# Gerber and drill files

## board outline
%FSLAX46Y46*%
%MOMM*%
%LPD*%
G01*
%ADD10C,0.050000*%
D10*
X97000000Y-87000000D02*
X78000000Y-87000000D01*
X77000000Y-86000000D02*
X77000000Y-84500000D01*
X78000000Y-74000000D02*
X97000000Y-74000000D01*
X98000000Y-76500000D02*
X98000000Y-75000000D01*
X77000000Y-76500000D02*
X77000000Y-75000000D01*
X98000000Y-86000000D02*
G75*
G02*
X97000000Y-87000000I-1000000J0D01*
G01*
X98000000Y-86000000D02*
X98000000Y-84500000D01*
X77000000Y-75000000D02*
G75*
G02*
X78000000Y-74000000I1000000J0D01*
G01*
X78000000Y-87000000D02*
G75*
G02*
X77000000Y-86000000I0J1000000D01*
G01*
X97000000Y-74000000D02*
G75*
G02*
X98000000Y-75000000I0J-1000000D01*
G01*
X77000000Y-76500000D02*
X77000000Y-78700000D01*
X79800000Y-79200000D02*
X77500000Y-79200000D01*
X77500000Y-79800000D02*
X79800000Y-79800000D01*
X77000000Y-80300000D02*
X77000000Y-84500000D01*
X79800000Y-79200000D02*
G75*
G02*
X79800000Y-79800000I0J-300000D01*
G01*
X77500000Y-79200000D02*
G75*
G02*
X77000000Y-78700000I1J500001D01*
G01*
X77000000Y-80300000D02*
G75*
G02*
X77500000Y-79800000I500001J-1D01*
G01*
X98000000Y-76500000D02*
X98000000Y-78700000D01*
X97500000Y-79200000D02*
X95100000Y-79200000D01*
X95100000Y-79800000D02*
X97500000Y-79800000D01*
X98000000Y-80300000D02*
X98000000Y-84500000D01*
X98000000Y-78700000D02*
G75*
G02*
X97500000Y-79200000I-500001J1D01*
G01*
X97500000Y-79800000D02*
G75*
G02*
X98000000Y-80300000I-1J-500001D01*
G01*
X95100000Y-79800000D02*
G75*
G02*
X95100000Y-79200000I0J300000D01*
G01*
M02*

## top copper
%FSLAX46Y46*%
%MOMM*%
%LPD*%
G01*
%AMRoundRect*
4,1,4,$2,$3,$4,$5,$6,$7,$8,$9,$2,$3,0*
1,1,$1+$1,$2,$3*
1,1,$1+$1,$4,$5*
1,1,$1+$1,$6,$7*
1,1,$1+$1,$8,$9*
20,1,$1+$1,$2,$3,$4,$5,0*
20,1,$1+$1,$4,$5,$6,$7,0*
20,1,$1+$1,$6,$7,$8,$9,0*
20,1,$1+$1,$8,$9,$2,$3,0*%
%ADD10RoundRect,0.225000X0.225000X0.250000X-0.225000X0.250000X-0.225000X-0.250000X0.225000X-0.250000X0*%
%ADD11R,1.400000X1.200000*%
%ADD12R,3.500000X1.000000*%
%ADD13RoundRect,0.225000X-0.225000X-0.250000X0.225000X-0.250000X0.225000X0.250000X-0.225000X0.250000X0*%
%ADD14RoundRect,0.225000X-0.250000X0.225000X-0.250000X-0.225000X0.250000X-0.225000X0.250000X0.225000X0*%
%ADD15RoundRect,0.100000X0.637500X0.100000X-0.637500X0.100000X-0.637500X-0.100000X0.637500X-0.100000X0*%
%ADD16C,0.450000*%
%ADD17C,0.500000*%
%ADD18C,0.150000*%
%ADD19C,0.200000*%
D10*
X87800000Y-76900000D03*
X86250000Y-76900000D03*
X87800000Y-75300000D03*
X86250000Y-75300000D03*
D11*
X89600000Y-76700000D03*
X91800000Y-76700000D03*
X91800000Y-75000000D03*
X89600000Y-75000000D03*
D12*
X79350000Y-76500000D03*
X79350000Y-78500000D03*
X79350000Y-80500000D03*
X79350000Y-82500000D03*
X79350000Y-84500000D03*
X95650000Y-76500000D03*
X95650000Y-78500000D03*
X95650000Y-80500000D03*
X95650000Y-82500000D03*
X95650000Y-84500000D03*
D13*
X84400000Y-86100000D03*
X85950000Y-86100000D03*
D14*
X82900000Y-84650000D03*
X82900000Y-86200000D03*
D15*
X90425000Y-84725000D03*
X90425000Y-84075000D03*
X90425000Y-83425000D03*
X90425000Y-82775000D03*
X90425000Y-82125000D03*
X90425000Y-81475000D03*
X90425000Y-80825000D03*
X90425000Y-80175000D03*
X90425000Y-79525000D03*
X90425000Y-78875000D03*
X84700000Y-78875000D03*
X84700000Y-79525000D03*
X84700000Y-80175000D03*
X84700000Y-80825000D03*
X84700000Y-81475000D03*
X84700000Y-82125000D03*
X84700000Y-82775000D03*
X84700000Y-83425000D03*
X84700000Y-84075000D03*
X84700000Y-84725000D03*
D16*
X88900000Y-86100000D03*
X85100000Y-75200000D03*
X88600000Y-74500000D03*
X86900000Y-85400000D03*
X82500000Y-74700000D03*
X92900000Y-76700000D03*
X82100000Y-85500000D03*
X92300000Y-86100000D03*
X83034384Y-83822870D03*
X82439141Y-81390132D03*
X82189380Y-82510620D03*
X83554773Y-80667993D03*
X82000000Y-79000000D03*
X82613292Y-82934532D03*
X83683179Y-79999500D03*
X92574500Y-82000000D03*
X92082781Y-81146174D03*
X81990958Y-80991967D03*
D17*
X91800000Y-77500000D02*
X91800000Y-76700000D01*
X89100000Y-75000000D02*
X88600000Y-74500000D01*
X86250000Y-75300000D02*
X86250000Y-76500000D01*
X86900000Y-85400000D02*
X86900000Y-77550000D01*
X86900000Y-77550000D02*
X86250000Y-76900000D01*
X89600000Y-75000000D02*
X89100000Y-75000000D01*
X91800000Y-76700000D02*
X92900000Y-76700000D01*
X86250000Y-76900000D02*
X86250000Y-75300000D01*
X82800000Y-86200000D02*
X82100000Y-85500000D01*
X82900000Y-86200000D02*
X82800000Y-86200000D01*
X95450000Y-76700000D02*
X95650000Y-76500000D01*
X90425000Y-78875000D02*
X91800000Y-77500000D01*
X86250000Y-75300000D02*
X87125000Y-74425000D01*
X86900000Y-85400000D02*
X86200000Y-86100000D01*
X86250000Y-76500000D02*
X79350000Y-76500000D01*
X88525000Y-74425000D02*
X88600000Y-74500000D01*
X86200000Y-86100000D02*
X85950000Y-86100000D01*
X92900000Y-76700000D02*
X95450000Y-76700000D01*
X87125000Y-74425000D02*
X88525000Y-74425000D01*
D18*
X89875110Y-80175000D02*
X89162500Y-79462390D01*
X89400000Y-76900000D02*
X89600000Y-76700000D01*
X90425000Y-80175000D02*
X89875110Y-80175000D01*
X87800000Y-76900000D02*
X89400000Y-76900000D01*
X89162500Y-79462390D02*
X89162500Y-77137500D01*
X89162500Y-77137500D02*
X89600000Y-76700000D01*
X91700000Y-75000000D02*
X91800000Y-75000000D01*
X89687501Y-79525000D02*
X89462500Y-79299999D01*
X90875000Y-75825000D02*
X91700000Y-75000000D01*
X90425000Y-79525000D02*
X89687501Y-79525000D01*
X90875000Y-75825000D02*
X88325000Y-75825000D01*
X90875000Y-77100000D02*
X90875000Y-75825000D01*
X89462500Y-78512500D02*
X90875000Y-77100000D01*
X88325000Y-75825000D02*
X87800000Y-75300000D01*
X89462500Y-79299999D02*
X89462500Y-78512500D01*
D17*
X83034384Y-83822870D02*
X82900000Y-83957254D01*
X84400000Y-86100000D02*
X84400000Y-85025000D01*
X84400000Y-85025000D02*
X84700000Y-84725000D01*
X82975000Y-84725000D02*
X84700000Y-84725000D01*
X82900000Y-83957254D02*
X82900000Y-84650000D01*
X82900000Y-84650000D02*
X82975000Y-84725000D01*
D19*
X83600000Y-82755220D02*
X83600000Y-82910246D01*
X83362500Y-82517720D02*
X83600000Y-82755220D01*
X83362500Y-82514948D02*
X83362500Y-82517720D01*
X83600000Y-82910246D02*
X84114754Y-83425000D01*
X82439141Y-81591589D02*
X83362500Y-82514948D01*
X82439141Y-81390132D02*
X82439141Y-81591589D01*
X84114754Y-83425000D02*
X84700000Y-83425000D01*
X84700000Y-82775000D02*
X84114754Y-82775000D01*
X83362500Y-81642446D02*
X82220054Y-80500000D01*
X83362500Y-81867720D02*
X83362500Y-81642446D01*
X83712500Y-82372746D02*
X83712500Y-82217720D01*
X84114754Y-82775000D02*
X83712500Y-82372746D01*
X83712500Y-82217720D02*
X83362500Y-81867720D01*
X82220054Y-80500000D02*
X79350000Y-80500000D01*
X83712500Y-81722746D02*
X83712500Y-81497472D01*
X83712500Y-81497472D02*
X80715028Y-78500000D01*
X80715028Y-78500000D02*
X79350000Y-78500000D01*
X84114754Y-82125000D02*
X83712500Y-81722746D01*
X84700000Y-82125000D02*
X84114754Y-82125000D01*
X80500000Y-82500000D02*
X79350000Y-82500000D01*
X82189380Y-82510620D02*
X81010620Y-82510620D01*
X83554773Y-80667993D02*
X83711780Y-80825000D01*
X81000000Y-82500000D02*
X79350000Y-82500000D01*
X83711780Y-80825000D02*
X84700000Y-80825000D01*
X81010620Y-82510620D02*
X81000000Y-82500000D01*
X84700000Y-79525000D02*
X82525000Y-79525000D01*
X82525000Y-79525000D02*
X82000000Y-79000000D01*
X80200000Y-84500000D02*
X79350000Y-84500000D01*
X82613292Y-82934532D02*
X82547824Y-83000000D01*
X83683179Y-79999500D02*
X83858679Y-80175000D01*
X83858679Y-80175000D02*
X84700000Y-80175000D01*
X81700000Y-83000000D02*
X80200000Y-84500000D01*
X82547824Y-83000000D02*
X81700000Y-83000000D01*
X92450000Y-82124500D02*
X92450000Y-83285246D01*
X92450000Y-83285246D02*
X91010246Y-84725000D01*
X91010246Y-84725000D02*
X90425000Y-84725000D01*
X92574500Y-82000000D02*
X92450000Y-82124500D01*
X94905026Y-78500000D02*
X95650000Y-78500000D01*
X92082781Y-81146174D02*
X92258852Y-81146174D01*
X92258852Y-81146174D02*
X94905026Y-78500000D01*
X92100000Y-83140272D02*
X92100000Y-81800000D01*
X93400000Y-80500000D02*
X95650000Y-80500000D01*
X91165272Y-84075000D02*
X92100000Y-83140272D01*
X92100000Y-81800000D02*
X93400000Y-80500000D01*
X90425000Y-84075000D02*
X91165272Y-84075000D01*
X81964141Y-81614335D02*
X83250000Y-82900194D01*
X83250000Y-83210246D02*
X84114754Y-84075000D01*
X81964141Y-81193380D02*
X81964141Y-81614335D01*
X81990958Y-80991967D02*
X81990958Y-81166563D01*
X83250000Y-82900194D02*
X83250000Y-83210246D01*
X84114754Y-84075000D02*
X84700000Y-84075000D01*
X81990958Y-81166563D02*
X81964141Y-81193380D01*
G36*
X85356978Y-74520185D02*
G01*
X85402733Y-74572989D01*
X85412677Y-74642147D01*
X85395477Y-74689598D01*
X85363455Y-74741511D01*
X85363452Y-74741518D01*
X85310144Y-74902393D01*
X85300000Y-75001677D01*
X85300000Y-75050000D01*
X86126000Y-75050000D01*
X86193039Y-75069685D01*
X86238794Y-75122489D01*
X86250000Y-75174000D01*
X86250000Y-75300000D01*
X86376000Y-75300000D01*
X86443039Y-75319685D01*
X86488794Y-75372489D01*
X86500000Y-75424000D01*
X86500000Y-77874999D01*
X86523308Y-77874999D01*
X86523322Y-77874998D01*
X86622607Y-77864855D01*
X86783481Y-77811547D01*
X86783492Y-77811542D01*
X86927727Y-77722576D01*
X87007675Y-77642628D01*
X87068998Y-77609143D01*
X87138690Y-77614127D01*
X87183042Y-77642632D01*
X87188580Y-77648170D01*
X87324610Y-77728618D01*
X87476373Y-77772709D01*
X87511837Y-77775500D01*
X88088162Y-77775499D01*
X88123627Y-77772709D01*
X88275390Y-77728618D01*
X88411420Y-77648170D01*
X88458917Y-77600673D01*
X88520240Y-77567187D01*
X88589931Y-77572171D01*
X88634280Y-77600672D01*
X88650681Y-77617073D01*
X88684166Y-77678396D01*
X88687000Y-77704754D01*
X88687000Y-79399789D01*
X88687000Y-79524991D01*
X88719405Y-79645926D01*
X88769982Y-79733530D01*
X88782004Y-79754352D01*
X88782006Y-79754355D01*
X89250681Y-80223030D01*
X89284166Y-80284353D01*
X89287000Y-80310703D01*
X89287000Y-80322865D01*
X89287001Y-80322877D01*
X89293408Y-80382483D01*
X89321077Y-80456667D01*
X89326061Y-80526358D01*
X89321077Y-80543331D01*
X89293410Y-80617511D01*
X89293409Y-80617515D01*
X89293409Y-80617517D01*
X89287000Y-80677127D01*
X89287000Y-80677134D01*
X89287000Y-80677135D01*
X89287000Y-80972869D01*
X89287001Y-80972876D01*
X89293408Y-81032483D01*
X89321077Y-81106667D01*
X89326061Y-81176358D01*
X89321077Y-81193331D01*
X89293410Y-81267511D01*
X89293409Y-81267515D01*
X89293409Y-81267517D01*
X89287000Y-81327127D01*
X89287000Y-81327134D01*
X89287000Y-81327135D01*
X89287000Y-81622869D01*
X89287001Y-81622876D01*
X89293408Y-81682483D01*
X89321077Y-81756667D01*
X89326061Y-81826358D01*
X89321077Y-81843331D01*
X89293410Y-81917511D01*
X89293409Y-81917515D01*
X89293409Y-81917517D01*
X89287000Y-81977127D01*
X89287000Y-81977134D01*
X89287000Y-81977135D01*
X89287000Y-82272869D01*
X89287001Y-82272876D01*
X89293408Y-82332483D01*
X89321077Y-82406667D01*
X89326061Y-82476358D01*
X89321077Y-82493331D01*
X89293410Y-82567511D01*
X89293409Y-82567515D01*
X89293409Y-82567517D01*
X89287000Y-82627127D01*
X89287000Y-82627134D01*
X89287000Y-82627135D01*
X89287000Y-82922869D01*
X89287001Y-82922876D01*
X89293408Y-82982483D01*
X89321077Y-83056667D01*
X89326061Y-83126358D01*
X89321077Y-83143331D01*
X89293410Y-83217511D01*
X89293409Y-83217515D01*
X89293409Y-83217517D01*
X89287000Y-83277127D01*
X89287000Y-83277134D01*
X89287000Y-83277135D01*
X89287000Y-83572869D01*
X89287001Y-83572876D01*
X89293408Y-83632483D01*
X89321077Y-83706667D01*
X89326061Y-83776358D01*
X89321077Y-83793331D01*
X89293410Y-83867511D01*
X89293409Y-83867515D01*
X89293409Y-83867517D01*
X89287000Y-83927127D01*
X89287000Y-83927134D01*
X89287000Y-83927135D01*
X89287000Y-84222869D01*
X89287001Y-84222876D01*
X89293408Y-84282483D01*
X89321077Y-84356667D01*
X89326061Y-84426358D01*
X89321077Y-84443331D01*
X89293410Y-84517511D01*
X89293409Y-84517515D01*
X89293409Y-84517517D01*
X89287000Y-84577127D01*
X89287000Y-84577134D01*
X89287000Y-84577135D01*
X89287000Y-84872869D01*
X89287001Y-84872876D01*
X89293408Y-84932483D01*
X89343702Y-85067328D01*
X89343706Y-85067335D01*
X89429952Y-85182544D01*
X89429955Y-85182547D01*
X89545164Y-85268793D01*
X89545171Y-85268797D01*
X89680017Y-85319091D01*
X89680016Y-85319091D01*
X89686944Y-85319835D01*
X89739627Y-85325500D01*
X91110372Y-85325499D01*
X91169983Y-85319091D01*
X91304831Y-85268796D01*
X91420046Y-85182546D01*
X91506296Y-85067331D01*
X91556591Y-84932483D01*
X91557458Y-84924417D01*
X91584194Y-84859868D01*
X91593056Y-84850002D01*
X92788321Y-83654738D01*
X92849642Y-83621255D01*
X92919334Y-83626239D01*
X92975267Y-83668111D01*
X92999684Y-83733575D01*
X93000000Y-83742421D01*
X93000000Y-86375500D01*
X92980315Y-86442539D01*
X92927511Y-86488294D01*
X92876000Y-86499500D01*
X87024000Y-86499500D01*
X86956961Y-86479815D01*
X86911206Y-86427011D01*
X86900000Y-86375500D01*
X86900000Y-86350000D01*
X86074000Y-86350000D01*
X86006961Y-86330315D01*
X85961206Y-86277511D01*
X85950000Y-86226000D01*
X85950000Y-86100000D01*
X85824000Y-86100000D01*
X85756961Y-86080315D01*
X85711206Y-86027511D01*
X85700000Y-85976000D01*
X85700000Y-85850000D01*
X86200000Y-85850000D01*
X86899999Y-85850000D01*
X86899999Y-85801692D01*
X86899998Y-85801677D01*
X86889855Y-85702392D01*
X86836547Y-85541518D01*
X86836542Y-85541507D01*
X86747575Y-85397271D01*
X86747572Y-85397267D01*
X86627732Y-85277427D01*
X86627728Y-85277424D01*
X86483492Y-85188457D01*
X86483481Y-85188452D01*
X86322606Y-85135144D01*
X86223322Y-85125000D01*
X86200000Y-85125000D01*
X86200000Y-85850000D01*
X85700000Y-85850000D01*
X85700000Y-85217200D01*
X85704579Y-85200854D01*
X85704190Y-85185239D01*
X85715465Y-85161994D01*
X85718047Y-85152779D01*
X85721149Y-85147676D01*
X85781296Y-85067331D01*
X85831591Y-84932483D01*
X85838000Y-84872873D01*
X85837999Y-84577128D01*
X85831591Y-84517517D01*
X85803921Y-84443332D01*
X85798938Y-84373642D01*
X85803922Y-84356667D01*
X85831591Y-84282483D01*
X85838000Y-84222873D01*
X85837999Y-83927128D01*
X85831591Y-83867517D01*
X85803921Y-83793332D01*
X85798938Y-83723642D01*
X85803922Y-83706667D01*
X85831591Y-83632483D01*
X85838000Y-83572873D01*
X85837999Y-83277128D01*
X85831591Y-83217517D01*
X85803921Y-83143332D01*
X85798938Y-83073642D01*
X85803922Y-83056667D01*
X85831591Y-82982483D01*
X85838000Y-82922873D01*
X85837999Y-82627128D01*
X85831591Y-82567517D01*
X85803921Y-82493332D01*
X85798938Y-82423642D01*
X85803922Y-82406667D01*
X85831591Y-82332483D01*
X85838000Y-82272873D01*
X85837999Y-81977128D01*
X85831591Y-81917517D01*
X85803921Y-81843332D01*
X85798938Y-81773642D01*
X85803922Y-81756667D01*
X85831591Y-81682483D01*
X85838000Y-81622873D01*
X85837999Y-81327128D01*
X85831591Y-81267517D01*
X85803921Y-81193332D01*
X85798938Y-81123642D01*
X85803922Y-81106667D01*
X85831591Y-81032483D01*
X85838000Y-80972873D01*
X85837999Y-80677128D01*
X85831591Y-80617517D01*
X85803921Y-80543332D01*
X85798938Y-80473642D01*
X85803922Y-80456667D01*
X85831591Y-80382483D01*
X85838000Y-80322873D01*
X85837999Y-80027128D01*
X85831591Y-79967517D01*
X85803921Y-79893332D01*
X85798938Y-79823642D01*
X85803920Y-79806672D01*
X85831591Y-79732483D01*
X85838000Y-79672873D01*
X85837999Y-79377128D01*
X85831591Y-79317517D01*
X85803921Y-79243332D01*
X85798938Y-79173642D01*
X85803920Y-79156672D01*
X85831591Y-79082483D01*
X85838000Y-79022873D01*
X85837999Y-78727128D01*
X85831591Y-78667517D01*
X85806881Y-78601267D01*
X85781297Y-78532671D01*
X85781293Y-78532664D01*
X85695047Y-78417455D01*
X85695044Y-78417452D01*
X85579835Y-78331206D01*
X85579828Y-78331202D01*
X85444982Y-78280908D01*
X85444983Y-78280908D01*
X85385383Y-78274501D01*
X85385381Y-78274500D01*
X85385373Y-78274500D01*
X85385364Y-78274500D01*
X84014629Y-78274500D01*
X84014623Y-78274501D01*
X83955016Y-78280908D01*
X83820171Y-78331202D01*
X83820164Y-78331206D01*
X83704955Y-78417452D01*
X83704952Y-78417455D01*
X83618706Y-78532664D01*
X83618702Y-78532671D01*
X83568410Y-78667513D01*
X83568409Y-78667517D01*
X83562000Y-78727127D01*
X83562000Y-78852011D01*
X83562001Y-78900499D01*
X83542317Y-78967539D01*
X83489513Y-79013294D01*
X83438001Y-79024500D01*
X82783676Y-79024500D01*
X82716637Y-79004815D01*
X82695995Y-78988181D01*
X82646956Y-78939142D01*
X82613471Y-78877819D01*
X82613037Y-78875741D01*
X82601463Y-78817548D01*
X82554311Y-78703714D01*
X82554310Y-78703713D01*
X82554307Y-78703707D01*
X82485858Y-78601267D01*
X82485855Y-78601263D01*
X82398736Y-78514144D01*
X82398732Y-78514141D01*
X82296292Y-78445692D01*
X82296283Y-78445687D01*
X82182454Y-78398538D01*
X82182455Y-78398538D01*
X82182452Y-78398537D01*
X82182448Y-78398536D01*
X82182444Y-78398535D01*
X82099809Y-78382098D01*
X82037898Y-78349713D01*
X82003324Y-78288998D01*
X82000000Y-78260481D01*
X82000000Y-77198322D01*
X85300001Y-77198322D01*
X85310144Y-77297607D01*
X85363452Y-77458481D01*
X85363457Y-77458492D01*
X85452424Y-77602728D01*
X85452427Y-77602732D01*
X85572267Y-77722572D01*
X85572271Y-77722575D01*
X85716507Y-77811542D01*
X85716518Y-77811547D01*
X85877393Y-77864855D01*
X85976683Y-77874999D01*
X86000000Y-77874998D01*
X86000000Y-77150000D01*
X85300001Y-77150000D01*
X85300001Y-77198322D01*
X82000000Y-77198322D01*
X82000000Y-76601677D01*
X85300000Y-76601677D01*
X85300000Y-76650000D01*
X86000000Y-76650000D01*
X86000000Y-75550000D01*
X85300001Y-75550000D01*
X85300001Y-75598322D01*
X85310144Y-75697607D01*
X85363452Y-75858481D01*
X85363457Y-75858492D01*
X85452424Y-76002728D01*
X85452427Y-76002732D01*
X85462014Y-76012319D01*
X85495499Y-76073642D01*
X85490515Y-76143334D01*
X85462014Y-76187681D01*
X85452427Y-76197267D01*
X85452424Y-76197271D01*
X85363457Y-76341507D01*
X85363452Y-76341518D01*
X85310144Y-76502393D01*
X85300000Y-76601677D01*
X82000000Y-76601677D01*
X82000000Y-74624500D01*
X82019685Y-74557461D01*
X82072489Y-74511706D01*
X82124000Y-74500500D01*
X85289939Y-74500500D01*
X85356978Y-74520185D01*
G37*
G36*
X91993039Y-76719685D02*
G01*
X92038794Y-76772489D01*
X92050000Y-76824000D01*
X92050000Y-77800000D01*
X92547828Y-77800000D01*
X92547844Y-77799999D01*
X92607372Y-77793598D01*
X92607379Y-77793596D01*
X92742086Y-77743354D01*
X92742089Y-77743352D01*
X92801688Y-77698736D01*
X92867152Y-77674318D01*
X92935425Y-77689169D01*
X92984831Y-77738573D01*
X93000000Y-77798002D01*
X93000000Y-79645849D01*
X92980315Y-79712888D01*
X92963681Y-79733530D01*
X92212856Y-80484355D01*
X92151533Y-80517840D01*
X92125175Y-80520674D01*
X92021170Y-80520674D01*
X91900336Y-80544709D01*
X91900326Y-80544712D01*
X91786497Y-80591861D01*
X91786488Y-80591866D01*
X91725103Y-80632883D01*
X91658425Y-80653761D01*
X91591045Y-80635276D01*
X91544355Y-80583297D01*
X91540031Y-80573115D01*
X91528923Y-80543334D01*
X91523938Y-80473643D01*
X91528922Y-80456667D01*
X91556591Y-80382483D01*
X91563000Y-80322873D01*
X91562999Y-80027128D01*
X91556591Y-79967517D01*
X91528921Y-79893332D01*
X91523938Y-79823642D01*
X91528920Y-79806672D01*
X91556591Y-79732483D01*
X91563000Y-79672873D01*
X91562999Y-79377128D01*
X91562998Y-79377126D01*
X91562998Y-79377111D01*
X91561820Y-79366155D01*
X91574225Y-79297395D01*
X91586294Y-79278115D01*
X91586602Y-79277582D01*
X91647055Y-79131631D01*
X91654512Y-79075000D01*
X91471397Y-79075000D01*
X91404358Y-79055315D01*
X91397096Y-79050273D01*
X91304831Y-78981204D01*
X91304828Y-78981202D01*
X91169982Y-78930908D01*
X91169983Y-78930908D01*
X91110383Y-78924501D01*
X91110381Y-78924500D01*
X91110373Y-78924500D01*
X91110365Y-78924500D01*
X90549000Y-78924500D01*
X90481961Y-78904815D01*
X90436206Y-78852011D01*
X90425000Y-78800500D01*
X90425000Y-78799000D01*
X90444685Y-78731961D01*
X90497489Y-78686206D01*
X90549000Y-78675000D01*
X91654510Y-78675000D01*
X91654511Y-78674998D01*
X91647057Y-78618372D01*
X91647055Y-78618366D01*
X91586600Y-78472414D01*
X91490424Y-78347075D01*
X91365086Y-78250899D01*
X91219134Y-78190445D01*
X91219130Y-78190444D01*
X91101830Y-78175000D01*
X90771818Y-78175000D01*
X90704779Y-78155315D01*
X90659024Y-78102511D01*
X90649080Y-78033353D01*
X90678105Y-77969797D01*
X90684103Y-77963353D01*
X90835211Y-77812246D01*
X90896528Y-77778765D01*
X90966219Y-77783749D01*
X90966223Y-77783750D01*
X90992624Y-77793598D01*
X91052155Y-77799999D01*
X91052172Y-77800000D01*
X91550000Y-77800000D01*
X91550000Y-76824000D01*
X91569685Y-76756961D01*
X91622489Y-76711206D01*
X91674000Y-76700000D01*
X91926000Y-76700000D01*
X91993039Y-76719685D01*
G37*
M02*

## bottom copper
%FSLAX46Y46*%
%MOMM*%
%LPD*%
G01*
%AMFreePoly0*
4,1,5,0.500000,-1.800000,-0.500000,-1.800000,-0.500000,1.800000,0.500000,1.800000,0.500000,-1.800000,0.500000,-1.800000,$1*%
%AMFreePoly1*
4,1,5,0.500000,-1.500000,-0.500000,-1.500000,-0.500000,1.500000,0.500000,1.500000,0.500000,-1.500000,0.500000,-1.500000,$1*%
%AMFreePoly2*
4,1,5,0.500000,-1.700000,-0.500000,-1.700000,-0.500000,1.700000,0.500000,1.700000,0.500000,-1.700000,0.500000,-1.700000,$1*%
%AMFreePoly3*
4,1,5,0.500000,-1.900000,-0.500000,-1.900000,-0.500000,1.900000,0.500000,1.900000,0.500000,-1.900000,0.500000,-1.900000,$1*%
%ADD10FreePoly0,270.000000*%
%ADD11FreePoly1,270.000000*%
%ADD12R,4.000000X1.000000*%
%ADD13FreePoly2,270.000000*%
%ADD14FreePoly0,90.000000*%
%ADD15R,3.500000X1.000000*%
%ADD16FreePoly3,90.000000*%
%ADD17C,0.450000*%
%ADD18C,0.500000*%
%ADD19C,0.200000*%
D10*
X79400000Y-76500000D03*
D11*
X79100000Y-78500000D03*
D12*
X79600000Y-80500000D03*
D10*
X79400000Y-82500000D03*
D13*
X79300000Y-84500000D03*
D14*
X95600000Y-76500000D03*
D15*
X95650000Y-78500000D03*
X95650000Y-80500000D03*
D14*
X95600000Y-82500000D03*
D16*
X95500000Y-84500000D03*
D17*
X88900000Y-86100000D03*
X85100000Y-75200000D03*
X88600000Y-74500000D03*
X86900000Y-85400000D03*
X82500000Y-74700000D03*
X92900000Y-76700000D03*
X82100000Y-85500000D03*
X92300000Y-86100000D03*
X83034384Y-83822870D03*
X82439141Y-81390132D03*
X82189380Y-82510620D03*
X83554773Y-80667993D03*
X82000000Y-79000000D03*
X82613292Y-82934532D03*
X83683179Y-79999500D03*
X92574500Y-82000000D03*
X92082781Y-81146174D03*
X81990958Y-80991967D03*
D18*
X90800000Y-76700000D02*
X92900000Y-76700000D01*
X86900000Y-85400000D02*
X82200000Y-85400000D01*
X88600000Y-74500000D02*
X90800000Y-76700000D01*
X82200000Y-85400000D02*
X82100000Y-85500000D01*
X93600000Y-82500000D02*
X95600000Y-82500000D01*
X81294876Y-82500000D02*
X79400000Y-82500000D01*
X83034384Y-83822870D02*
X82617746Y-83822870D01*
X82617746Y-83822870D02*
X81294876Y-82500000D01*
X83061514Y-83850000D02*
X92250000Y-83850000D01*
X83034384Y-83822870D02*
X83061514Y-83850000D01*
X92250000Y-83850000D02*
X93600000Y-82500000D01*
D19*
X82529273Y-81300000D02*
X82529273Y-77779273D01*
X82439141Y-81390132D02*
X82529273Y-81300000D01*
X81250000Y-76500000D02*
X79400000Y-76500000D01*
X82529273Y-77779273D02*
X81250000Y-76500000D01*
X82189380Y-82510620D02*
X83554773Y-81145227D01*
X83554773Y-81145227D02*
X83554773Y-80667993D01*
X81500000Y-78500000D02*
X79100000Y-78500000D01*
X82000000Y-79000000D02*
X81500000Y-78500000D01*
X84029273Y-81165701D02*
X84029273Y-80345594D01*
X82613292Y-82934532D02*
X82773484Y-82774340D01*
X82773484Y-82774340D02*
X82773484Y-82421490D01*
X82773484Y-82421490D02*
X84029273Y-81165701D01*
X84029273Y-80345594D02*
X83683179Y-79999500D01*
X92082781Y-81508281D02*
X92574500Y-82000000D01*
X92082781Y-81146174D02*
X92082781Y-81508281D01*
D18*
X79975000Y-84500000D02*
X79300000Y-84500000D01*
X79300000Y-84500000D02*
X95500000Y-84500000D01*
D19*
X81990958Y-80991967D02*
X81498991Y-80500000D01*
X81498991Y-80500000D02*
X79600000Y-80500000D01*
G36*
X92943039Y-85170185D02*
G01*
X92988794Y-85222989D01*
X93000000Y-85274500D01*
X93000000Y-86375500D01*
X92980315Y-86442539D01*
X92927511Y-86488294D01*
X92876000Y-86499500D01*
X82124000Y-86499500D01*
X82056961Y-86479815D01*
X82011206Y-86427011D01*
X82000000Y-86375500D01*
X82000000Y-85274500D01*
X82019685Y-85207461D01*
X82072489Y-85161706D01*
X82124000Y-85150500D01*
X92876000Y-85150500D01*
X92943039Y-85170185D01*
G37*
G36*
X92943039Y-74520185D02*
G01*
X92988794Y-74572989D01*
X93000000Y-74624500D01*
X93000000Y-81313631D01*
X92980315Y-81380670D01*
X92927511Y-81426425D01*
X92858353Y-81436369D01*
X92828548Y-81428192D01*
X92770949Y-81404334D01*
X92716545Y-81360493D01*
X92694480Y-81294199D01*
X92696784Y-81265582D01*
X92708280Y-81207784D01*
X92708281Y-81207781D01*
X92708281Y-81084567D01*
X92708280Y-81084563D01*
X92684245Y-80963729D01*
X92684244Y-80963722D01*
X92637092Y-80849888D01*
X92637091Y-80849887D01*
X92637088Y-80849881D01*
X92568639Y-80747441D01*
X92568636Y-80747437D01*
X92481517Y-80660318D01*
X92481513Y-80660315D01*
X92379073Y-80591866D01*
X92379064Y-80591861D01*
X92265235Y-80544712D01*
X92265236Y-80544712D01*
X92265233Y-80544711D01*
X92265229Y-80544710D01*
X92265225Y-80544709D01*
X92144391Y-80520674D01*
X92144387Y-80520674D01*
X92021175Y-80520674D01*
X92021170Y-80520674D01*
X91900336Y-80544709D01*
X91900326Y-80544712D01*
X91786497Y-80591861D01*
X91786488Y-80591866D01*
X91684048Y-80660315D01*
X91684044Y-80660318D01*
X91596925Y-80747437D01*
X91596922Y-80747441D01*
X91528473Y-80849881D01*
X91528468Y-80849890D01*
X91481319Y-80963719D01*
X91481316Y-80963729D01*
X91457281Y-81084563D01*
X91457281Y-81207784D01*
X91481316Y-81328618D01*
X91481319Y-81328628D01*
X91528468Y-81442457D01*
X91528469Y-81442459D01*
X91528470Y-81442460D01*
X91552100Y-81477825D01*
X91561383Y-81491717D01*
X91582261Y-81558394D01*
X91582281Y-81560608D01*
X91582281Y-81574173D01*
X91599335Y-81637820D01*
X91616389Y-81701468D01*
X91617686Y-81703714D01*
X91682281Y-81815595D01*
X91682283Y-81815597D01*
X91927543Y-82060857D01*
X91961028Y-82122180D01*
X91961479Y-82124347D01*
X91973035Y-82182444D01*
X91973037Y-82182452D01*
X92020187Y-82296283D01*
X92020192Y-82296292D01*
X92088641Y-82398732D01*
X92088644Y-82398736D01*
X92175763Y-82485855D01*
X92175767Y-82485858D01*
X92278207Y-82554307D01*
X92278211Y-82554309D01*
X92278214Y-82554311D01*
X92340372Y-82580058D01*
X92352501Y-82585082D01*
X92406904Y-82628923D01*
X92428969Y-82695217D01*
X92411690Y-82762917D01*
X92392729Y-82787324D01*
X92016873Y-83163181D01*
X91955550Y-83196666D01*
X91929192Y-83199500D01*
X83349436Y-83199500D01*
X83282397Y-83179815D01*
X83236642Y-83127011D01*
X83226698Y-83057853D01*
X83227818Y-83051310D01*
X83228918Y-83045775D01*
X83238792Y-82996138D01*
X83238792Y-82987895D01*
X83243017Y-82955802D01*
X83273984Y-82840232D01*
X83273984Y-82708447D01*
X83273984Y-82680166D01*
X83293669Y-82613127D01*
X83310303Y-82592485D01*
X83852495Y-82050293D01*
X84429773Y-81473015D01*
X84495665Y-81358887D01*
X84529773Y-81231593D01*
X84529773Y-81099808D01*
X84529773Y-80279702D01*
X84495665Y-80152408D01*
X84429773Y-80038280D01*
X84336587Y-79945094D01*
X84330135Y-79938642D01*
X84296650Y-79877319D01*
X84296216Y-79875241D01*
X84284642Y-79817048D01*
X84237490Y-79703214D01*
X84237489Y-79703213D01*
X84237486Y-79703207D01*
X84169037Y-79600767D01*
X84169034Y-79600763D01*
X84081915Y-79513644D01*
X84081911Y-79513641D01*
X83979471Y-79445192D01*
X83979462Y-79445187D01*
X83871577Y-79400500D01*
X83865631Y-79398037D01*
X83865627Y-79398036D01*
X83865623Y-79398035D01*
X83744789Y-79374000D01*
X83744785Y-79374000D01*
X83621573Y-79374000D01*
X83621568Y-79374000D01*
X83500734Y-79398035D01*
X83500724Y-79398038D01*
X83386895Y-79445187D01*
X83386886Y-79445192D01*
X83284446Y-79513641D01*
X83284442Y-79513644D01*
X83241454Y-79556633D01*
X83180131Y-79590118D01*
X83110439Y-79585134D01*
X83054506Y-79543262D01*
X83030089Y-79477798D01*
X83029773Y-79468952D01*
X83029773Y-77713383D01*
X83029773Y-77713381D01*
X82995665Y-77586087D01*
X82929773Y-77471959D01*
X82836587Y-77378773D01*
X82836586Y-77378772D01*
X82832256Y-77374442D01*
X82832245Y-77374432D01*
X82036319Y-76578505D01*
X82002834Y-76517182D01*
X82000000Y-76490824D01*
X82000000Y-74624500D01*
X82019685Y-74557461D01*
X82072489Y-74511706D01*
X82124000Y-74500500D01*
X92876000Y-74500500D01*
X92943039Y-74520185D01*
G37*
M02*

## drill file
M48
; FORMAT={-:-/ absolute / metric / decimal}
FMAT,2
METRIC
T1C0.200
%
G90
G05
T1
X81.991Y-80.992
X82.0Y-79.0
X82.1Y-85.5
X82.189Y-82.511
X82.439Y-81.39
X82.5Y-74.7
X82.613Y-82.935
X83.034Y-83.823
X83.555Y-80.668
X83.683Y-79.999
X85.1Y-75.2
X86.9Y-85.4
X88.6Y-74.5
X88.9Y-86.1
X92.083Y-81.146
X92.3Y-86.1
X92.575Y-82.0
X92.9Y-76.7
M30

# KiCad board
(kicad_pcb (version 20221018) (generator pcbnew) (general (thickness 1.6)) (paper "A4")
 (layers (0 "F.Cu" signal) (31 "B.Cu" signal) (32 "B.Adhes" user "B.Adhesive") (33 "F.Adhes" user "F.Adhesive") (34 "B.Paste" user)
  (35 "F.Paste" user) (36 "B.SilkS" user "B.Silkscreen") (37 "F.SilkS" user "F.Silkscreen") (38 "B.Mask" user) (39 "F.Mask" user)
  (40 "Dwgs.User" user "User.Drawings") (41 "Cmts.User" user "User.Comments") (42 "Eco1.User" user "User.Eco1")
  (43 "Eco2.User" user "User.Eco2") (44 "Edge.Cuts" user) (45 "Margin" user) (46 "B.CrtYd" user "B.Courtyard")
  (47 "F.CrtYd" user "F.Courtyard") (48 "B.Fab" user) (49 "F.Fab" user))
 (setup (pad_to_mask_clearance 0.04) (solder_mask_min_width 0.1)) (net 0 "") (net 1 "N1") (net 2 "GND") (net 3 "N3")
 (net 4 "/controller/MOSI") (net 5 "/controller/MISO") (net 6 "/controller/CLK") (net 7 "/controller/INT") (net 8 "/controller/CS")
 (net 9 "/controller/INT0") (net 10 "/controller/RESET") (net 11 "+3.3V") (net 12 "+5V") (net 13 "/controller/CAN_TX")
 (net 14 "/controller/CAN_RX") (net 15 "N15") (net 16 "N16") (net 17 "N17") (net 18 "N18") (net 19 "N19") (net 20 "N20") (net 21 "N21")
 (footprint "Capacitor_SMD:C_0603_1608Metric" (layer "F.Cu") (at 87.025 76.9 180)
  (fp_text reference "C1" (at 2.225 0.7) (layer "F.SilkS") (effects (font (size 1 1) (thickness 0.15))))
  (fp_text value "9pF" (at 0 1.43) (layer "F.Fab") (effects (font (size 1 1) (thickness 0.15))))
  (pad "1" smd roundrect (at -0.775 0 180) (size 0.9 0.95) (layers "F.Cu" "F.Paste" "F.Mask") (roundrect_rratio 0.25) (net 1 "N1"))
  (pad "2" smd roundrect (at 0.775 0 180) (size 0.9 0.95) (layers "F.Cu" "F.Paste" "F.Mask") (roundrect_rratio 0.25) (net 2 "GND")))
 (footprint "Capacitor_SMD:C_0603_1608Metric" (layer "F.Cu") (at 87.025 75.3 180)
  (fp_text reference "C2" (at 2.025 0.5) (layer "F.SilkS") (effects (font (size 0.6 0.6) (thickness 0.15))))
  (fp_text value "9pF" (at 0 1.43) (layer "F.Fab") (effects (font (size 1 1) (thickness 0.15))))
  (pad "1" smd roundrect (at -0.775 0 180) (size 0.9 0.95) (layers "F.Cu" "F.Paste" "F.Mask") (roundrect_rratio 0.25) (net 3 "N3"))
  (pad "2" smd roundrect (at 0.775 0 180) (size 0.9 0.95) (layers "F.Cu" "F.Paste" "F.Mask") (roundrect_rratio 0.25) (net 2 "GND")))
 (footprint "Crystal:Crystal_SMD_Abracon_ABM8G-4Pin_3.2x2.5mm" (layer "F.Cu") (at 90.7 75.85)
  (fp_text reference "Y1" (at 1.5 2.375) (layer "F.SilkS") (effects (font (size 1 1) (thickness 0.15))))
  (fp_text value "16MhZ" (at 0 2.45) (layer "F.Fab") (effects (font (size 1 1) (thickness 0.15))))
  (pad "1" smd rect (at -1.1 0.85) (size 1.4 1.2) (layers "F.Cu" "F.Paste" "F.Mask") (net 1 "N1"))
  (pad "2" smd rect (at 1.1 0.85) (size 1.4 1.2) (layers "F.Cu" "F.Paste" "F.Mask") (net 2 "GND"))
  (pad "3" smd rect (at 1.1 -0.85) (size 1.4 1.2) (layers "F.Cu" "F.Paste" "F.Mask") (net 3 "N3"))
  (pad "4" smd rect (at -1.1 -0.85) (size 1.4 1.2) (layers "F.Cu" "F.Paste" "F.Mask") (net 2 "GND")))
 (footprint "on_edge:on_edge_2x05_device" (layer "F.Cu") (at 77 80.5 -90)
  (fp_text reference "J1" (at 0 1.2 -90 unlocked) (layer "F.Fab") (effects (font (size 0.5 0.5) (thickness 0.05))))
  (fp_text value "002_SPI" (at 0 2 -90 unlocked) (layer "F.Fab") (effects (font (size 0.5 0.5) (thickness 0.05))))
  (fp_line (start -4 0) (end -1.8 0) (stroke (width 0.05) (type solid)) (layer "Edge.Cuts"))
  (fp_line (start -1.3 -2.8) (end -1.3 -0.5) (stroke (width 0.05) (type solid)) (layer "Edge.Cuts"))
  (fp_line (start -0.7 -0.5) (end -0.7 -2.8) (stroke (width 0.05) (type solid)) (layer "Edge.Cuts"))
  (fp_line (start -0.2 0) (end 4 0) (stroke (width 0.05) (type solid)) (layer "Edge.Cuts"))
  (fp_arc (start -1.3 -2.8) (mid -1 -3.1) (end -0.7 -2.8) (stroke (width 0.05) (type solid)) (layer "Edge.Cuts"))
  (fp_arc (start -1.3 -0.5) (mid -1.446447 -0.146447) (end -1.8 0) (stroke (width 0.05) (type solid)) (layer "Edge.Cuts"))
  (fp_arc (start -0.2 0) (mid -0.553553 -0.146447) (end -0.7 -0.5) (stroke (width 0.05) (type solid)) (layer "Edge.Cuts"))
  (pad "1" smd rect (at -4 -2.35 90) (size 1 3.5) (layers "F.Cu" "F.Mask") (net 2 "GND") (zone_connect 0))
  (pad "2" smd rect (at -2 -2.35 270) (size 1 3.5) (layers "F.Cu" "F.Mask") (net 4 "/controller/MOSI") (zone_connect 0))
  (pad "3" smd rect (at 0 -2.35 270) (size 1 3.5) (layers "F.Cu" "F.Mask") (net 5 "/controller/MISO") (zone_connect 0))
  (pad "4" smd rect (at 2 -2.35 90) (size 1 3.5) (layers "F.Cu" "F.Mask") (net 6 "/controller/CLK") (zone_connect 0))
  (pad "5" smd rect (at 4 -2.35 90) (size 1 3.5) (layers "F.Cu" "F.Mask") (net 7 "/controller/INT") (zone_connect 0))
  (pad "6" smd custom (at -4 -2.4 270) (size 1 3.6) (layers "B.Cu" "B.Mask") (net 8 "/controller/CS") (zone_connect 0)
   (options (clearance outline) (anchor rect)) (primitives))
  (pad "7" smd custom (at -2 -2.1 270) (size 1 3) (layers "B.Cu" "B.Mask") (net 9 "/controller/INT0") (zone_connect 0)
   (options (clearance outline) (anchor rect)) (primitives))
  (pad "8" smd rect (at 0 -2.6 270) (size 1 4) (layers "B.Cu" "B.Mask") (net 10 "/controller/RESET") (zone_connect 0))
  (pad "9" smd custom (at 2 -2.4 270) (size 1 3.6) (layers "B.Cu" "B.Mask") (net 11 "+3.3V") (zone_connect 0)
   (options (clearance outline) (anchor rect)) (primitives))
  (pad "10" smd custom (at 4 -2.3 270) (size 1 3.4) (layers "B.Cu" "B.Mask") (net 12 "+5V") (zone_connect 0)
   (options (clearance outline) (anchor rect)) (primitives))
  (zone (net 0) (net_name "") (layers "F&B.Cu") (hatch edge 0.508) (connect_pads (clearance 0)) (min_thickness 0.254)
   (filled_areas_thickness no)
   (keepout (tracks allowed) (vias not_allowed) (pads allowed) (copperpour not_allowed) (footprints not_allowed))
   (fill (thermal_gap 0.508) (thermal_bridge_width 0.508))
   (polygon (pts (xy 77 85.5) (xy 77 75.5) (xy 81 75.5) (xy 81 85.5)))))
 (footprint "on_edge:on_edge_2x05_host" (layer "F.Cu") (at 98 80.5 -90)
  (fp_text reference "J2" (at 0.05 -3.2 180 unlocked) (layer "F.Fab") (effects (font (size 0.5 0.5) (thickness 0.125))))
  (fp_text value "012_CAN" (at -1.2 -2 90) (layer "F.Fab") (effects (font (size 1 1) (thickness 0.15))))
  (fp_line (start -4 0) (end -1.8 0) (stroke (width 0.05) (type solid)) (layer "Edge.Cuts"))
  (fp_line (start -1.3 0.5) (end -1.3 2.9) (stroke (width 0.05) (type solid)) (layer "Edge.Cuts"))
  (fp_line (start -0.7 2.9) (end -0.7 0.5) (stroke (width 0.05) (type solid)) (layer "Edge.Cuts"))
  (fp_line (start -0.2 0) (end 4 0) (stroke (width 0.05) (type solid)) (layer "Edge.Cuts"))
  (fp_arc (start -1.8 0) (mid -1.446447 0.146447) (end -1.3 0.5) (stroke (width 0.05) (type solid)) (layer "Edge.Cuts"))
  (fp_arc (start -0.7 0.5) (mid -0.553553 0.146447) (end -0.2 0) (stroke (width 0.05) (type solid)) (layer "Edge.Cuts"))
  (fp_arc (start -0.7 2.9) (mid -1 3.2) (end -1.3 2.9) (stroke (width 0.05) (type solid)) (layer "Edge.Cuts"))
  (pad "1" smd rect (at -4 2.35 270) (size 1 3.5) (layers "F.Cu" "F.Mask") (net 2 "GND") (zone_connect 0))
  (pad "2" smd rect (at -2 2.35 270) (size 1 3.5) (layers "F.Cu" "F.Mask") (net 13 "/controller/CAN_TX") (zone_connect 0))
  (pad "3" smd rect (at 0 2.35 270) (size 1 3.5) (layers "F.Cu" "F.Mask") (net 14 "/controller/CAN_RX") (zone_connect 0))
  (pad "4" smd rect (at 2 2.35 270) (size 1 3.5) (layers "F.Cu" "F.Mask") (zone_connect 0))
  (pad "5" smd rect (at 4 2.35 270) (size 1 3.5) (layers "F.Cu" "F.Mask") (zone_connect 0))
  (pad "6" smd custom (at -4 2.4 90) (size 1 3.6) (layers "B.Cu" "B.Mask") (zone_connect 0) (options (clearance outline) (anchor rect))
   (primitives))
  (pad "7" smd rect (at -2 2.35 90) (size 1 3.5) (layers "B.Cu" "B.Mask") (zone_connect 0))
  (pad "8" smd rect (at 0 2.35 90) (size 1 3.5) (layers "B.Cu" "B.Mask") (zone_connect 0))
  (pad "9" smd custom (at 2 2.4 90) (size 1 3.6) (layers "B.Cu" "B.Mask") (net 11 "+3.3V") (zone_connect 0)
   (options (clearance outline) (anchor rect)) (primitives))
  (pad "10" smd custom (at 4 2.5 90) (size 1 3.8) (layers "B.Cu" "B.Mask") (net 12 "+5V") (zone_connect 0)
   (options (clearance outline) (anchor rect)) (primitives))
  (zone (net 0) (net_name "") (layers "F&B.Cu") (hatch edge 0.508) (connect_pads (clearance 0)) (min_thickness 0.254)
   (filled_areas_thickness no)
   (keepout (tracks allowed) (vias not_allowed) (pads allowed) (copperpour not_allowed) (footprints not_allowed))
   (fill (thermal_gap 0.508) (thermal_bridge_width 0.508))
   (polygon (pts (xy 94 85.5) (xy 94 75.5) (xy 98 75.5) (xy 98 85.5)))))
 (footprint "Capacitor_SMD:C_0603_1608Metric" (layer "F.Cu") (at 85.175 86.1)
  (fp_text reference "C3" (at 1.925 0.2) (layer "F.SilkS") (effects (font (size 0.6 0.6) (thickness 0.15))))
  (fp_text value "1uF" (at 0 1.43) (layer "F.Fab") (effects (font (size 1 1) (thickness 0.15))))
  (pad "1" smd roundrect (at -0.775 0) (size 0.9 0.95) (layers "F.Cu" "F.Paste" "F.Mask") (roundrect_rratio 0.25) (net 11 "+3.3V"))
  (pad "2" smd roundrect (at 0.775 0) (size 0.9 0.95) (layers "F.Cu" "F.Paste" "F.Mask") (roundrect_rratio 0.25) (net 2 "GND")))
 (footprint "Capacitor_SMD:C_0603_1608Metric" (layer "F.Cu") (at 82.9 85.425 -90)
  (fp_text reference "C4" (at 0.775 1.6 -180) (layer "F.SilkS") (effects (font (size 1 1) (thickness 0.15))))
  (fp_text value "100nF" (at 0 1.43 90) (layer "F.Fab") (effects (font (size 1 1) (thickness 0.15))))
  (pad "1" smd roundrect (at -0.775 0 270) (size 0.9 0.95) (layers "F.Cu" "F.Paste" "F.Mask") (roundrect_rratio 0.25) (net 11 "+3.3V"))
  (pad "2" smd roundrect (at 0.775 0 270) (size 0.9 0.95) (layers "F.Cu" "F.Paste" "F.Mask") (roundrect_rratio 0.25) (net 2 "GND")))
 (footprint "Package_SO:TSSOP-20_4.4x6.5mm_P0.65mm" (layer "F.Cu") (at 87.5625 81.8 180)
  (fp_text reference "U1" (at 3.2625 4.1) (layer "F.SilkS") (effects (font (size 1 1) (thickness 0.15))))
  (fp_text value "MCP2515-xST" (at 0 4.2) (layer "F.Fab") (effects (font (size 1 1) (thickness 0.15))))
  (pad "1" smd roundrect (at -2.8625 -2.925 180) (size 1.475 0.4) (layers "F.Cu" "F.Paste" "F.Mask") (roundrect_rratio 0.25)
   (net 13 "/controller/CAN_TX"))
  (pad "2" smd roundrect (at -2.8625 -2.275 180) (size 1.475 0.4) (layers "F.Cu" "F.Paste" "F.Mask") (roundrect_rratio 0.25)
   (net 14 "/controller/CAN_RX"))
  (pad "3" smd roundrect (at -2.8625 -1.625 180) (size 1.475 0.4) (layers "F.Cu" "F.Paste" "F.Mask") (roundrect_rratio 0.25) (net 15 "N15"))
  (pad "4" smd roundrect (at -2.8625 -0.975 180) (size 1.475 0.4) (layers "F.Cu" "F.Paste" "F.Mask") (roundrect_rratio 0.25) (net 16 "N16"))
  (pad "5" smd roundrect (at -2.8625 -0.325 180) (size 1.475 0.4) (layers "F.Cu" "F.Paste" "F.Mask") (roundrect_rratio 0.25) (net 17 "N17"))
  (pad "6" smd roundrect (at -2.8625 0.325 180) (size 1.475 0.4) (layers "F.Cu" "F.Paste" "F.Mask") (roundrect_rratio 0.25) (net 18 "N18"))
  (pad "7" smd roundrect (at -2.8625 0.975 180) (size 1.475 0.4) (layers "F.Cu" "F.Paste" "F.Mask") (roundrect_rratio 0.25) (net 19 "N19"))
  (pad "8" smd roundrect (at -2.8625 1.625 180) (size 1.475 0.4) (layers "F.Cu" "F.Paste" "F.Mask") (roundrect_rratio 0.25) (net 1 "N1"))
  (pad "9" smd roundrect (at -2.8625 2.275 180) (size 1.475 0.4) (layers "F.Cu" "F.Paste" "F.Mask") (roundrect_rratio 0.25) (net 3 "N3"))
  (pad "10" smd roundrect (at -2.8625 2.925 180) (size 1.475 0.4) (layers "F.Cu" "F.Paste" "F.Mask") (roundrect_rratio 0.25) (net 2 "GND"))
  (pad "11" smd roundrect (at 2.8625 2.925 180) (size 1.475 0.4) (layers "F.Cu" "F.Paste" "F.Mask") (roundrect_rratio 0.25) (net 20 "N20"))
  (pad "12" smd roundrect (at 2.8625 2.275 180) (size 1.475 0.4) (layers "F.Cu" "F.Paste" "F.Mask") (roundrect_rratio 0.25)
   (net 9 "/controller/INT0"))
  (pad "13" smd roundrect (at 2.8625 1.625 180) (size 1.475 0.4) (layers "F.Cu" "F.Paste" "F.Mask") (roundrect_rratio 0.25)
   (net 7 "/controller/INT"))
  (pad "14" smd roundrect (at 2.8625 0.975 180) (size 1.475 0.4) (layers "F.Cu" "F.Paste" "F.Mask") (roundrect_rratio 0.25)
   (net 6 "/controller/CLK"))
  (pad "15" smd roundrect (at 2.8625 0.325 180) (size 1.475 0.4) (layers "F.Cu" "F.Paste" "F.Mask") (roundrect_rratio 0.25) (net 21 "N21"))
  (pad "16" smd roundrect (at 2.8625 -0.325 180) (size 1.475 0.4) (layers "F.Cu" "F.Paste" "F.Mask") (roundrect_rratio 0.25)
   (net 4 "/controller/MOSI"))
  (pad "17" smd roundrect (at 2.8625 -0.975 180) (size 1.475 0.4) (layers "F.Cu" "F.Paste" "F.Mask") (roundrect_rratio 0.25)
   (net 5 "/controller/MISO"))
  (pad "18" smd roundrect (at 2.8625 -1.625 180) (size 1.475 0.4) (layers "F.Cu" "F.Paste" "F.Mask") (roundrect_rratio 0.25)
   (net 8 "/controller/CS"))
  (pad "19" smd roundrect (at 2.8625 -2.275 180) (size 1.475 0.4) (layers "F.Cu" "F.Paste" "F.Mask") (roundrect_rratio 0.25)
   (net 10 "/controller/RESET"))
  (pad "20" smd roundrect (at 2.8625 -2.925 180) (size 1.475 0.4) (layers "F.Cu" "F.Paste" "F.Mask") (roundrect_rratio 0.25)
   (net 11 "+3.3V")))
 (gr_line (start 97 87) (end 78 87) (stroke (width 0.05) (type solid)) (layer "Edge.Cuts"))
 (gr_line (start 77 86) (end 77 84.5) (stroke (width 0.05) (type solid)) (layer "Edge.Cuts"))
 (gr_line (start 78 74) (end 97 74) (stroke (width 0.05) (type solid)) (layer "Edge.Cuts"))
 (gr_line (start 98 76.5) (end 98 75) (stroke (width 0.05) (type solid)) (layer "Edge.Cuts"))
 (gr_line (start 77 76.5) (end 77 75) (stroke (width 0.05) (type solid)) (layer "Edge.Cuts"))
 (gr_arc (start 98 86) (mid 97.707107 86.707107) (end 97 87) (stroke (width 0.05) (type solid)) (layer "Edge.Cuts"))
 (gr_line (start 98 86) (end 98 84.5) (stroke (width 0.05) (type solid)) (layer "Edge.Cuts"))
 (gr_arc (start 77 75) (mid 77.292893 74.292893) (end 78 74) (stroke (width 0.05) (type solid)) (layer "Edge.Cuts"))
 (gr_arc (start 78 87) (mid 77.292893 86.707107) (end 77 86) (stroke (width 0.05) (type solid)) (layer "Edge.Cuts"))
 (gr_arc (start 97 74) (mid 97.707107 74.292893) (end 98 75) (stroke (width 0.05) (type solid)) (layer "Edge.Cuts"))
 (segment (start 91.8 77.5) (end 91.8 76.7) (width 0.5) (layer "F.Cu") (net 2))
 (segment (start 89.1 75) (end 88.6 74.5) (width 0.5) (layer "F.Cu") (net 2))
 (segment (start 86.25 75.3) (end 86.25 76.5) (width 0.5) (layer "F.Cu") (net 2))
 (segment (start 86.9 85.4) (end 86.9 77.55) (width 0.5) (layer "F.Cu") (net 2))
 (segment (start 86.9 77.55) (end 86.25 76.9) (width 0.5) (layer "F.Cu") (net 2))
 (segment (start 89.6 75) (end 89.1 75) (width 0.5) (layer "F.Cu") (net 2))
 (segment (start 91.8 76.7) (end 92.9 76.7) (width 0.5) (layer "F.Cu") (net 2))
 (segment (start 86.25 76.9) (end 86.25 75.3) (width 0.5) (layer "F.Cu") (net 2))
 (segment (start 82.8 86.2) (end 82.1 85.5) (width 0.5) (layer "F.Cu") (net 2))
 (segment (start 82.9 86.2) (end 82.8 86.2) (width 0.5) (layer "F.Cu") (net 2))
 (segment (start 95.45 76.7) (end 95.65 76.5) (width 0.5) (layer "F.Cu") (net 2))
 (segment (start 90.425 78.875) (end 91.8 77.5) (width 0.5) (layer "F.Cu") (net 2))
 (segment (start 86.25 75.3) (end 87.125 74.425) (width 0.5) (layer "F.Cu") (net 2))
 (segment (start 86.9 85.4) (end 86.2 86.1) (width 0.5) (layer "F.Cu") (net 2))
 (segment (start 86.25 76.5) (end 79.35 76.5) (width 0.5) (layer "F.Cu") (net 2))
 (segment (start 88.525 74.425) (end 88.6 74.5) (width 0.5) (layer "F.Cu") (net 2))
 (segment (start 86.2 86.1) (end 85.95 86.1) (width 0.5) (layer "F.Cu") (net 2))
 (segment (start 92.9 76.7) (end 95.45 76.7) (width 0.5) (layer "F.Cu") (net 2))
 (segment (start 87.125 74.425) (end 88.525 74.425) (width 0.5) (layer "F.Cu") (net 2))
 (via (at 88.9 86.1) (size 0.45) (drill 0.2) (layers "F.Cu" "B.Cu") (free) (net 2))
 (via (at 85.1 75.2) (size 0.45) (drill 0.2) (layers "F.Cu" "B.Cu") (free) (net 2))
 (via (at 88.6 74.5) (size 0.45) (drill 0.2) (layers "F.Cu" "B.Cu") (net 2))
 (via (at 86.9 85.4) (size 0.45) (drill 0.2) (layers "F.Cu" "B.Cu") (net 2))
 (via (at 82.5 74.7) (size 0.45) (drill 0.2) (layers "F.Cu" "B.Cu") (free) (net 2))
 (via (at 92.9 76.7) (size 0.45) (drill 0.2) (layers "F.Cu" "B.Cu") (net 2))
 (via (at 82.1 85.5) (size 0.45) (drill 0.2) (layers "F.Cu" "B.Cu") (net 2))
 (via (at 92.3 86.1) (size 0.45) (drill 0.2) (layers "F.Cu" "B.Cu") (free) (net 2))
 (segment (start 90.8 76.7) (end 92.9 76.7) (width 0.5) (layer "B.Cu") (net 2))
 (segment (start 86.9 85.4) (end 82.2 85.4) (width 0.5) (layer "B.Cu") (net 2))
 (segment (start 88.6 74.5) (end 90.8 76.7) (width 0.5) (layer "B.Cu") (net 2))
 (segment (start 82.2 85.4) (end 82.1 85.5) (width 0.5) (layer "B.Cu") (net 2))
 (segment (start 89.87511 80.175) (end 89.1625 79.46239) (width 0.15) (layer "F.Cu") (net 1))
 (segment (start 89.4 76.9) (end 89.6 76.7) (width 0.15) (layer "F.Cu") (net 1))
 (segment (start 90.425 80.175) (end 89.87511 80.175) (width 0.15) (layer "F.Cu") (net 1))
 (segment (start 87.8 76.9) (end 89.4 76.9) (width 0.15) (layer "F.Cu") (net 1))
 (segment (start 89.1625 79.46239) (end 89.1625 77.1375) (width 0.15) (layer "F.Cu") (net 1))
 (segment (start 89.1625 77.1375) (end 89.6 76.7) (width 0.15) (layer "F.Cu") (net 1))
 (segment (start 91.7 75) (end 91.8 75) (width 0.15) (layer "F.Cu") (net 3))
 (segment (start 89.687501 79.525) (end 89.4625 79.299999) (width 0.15) (layer "F.Cu") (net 3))
 (segment (start 90.875 75.825) (end 91.7 75) (width 0.15) (layer "F.Cu") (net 3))
 (segment (start 90.425 79.525) (end 89.687501 79.525) (width 0.15) (layer "F.Cu") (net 3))
 (segment (start 90.875 75.825) (end 88.325 75.825) (width 0.15) (layer "F.Cu") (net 3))
 (segment (start 90.875 77.1) (end 90.875 75.825) (width 0.15) (layer "F.Cu") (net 3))
 (segment (start 89.4625 78.5125) (end 90.875 77.1) (width 0.15) (layer "F.Cu") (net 3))
 (segment (start 88.325 75.825) (end 87.8 75.3) (width 0.15) (layer "F.Cu") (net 3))
 (segment (start 89.4625 79.299999) (end 89.4625 78.5125) (width 0.15) (layer "F.Cu") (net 3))
 (segment (start 83.034384 83.82287) (end 82.9 83.957254) (width 0.5) (layer "F.Cu") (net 11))
 (segment (start 84.4 86.1) (end 84.4 85.025) (width 0.5) (layer "F.Cu") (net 11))
 (segment (start 84.4 85.025) (end 84.7 84.725) (width 0.5) (layer "F.Cu") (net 11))
 (segment (start 82.975 84.725) (end 84.7 84.725) (width 0.5) (layer "F.Cu") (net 11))
 (segment (start 82.9 83.957254) (end 82.9 84.65) (width 0.5) (layer "F.Cu") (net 11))
 (segment (start 82.9 84.65) (end 82.975 84.725) (width 0.5) (layer "F.Cu") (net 11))
 (via (at 83.034384 83.82287) (size 0.45) (drill 0.2) (layers "F.Cu" "B.Cu") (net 11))
 (segment (start 93.6 82.5) (end 95.6 82.5) (width 0.5) (layer "B.Cu") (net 11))
 (segment (start 81.294876 82.5) (end 79.4 82.5) (width 0.5) (layer "B.Cu") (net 11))
 (segment (start 83.034384 83.82287) (end 82.617746 83.82287) (width 0.5) (layer "B.Cu") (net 11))
 (segment (start 82.617746 83.82287) (end 81.294876 82.5) (width 0.5) (layer "B.Cu") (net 11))
 (segment (start 83.061514 83.85) (end 92.25 83.85) (width 0.5) (layer "B.Cu") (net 11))
 (segment (start 83.034384 83.82287) (end 83.061514 83.85) (width 0.5) (layer "B.Cu") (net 11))
 (segment (start 92.25 83.85) (end 93.6 82.5) (width 0.5) (layer "B.Cu") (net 11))
 (segment (start 83.6 82.75522) (end 83.6 82.910246) (width 0.2) (layer "F.Cu") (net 8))
 (segment (start 83.3625 82.51772) (end 83.6 82.75522) (width 0.2) (layer "F.Cu") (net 8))
 (segment (start 83.3625 82.514948) (end 83.3625 82.51772) (width 0.2) (layer "F.Cu") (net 8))
 (segment (start 83.6 82.910246) (end 84.114754 83.425) (width 0.2) (layer "F.Cu") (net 8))
 (segment (start 82.439141 81.591589) (end 83.3625 82.514948) (width 0.2) (layer "F.Cu") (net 8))
 (segment (start 82.439141 81.390132) (end 82.439141 81.591589) (width 0.2) (layer "F.Cu") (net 8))
 (segment (start 84.114754 83.425) (end 84.7 83.425) (width 0.2) (layer "F.Cu") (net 8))
 (via (at 82.439141 81.390132) (size 0.45) (drill 0.2) (layers "F.Cu" "B.Cu") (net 8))
 (segment (start 82.529273 81.3) (end 82.529273 77.779273) (width 0.2) (layer "B.Cu") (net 8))
 (segment (start 82.439141 81.390132) (end 82.529273 81.3) (width 0.2) (layer "B.Cu") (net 8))
 (segment (start 81.25 76.5) (end 79.4 76.5) (width 0.2) (layer "B.Cu") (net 8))
 (segment (start 82.529273 77.779273) (end 81.25 76.5) (width 0.2) (layer "B.Cu") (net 8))
 (segment (start 84.7 82.775) (end 84.114754 82.775) (width 0.2) (layer "F.Cu") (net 5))
 (segment (start 83.3625 81.642446) (end 82.220054 80.5) (width 0.2) (layer "F.Cu") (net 5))
 (segment (start 83.3625 81.86772) (end 83.3625 81.642446) (width 0.2) (layer "F.Cu") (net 5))
 (segment (start 83.7125 82.372746) (end 83.7125 82.21772) (width 0.2) (layer "F.Cu") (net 5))
 (segment (start 84.114754 82.775) (end 83.7125 82.372746) (width 0.2) (layer "F.Cu") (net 5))
 (segment (start 83.7125 82.21772) (end 83.3625 81.86772) (width 0.2) (layer "F.Cu") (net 5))
 (segment (start 82.220054 80.5) (end 79.35 80.5) (width 0.2) (layer "F.Cu") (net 5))
 (segment (start 83.7125 81.722746) (end 83.7125 81.497472) (width 0.2) (layer "F.Cu") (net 4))
 (segment (start 83.7125 81.497472) (end 80.715028 78.5) (width 0.2) (layer "F.Cu") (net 4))
 (segment (start 80.715028 78.5) (end 79.35 78.5) (width 0.2) (layer "F.Cu") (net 4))
 (segment (start 84.114754 82.125) (end 83.7125 81.722746) (width 0.2) (layer "F.Cu") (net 4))
 (segment (start 84.7 82.125) (end 84.114754 82.125) (width 0.2) (layer "F.Cu") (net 4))
 (segment (start 80.5 82.5) (end 79.35 82.5) (width 0.2) (layer "F.Cu") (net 6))
 (segment (start 82.18938 82.51062) (end 81.01062 82.51062) (width 0.2) (layer "F.Cu") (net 6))
 (segment (start 83.554773 80.667993) (end 83.71178 80.825) (width 0.2) (layer "F.Cu") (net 6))
 (segment (start 81 82.5) (end 79.35 82.5) (width 0.2) (layer "F.Cu") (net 6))
 (segment (start 83.71178 80.825) (end 84.7 80.825) (width 0.2) (layer "F.Cu") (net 6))
 (segment (start 81.01062 82.51062) (end 81 82.5) (width 0.2) (layer "F.Cu") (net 6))
 (via (at 82.18938 82.51062) (size 0.45) (drill 0.2) (layers "F.Cu" "B.Cu") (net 6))
 (via (at 83.554773 80.667993) (size 0.45) (drill 0.2) (layers "F.Cu" "B.Cu") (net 6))
 (segment (start 82.18938 82.51062) (end 83.554773 81.145227) (width 0.2) (layer "B.Cu") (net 6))
 (segment (start 83.554773 81.145227) (end 83.554773 80.667993) (width 0.2) (layer "B.Cu") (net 6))
 (segment (start 84.7 79.525) (end 82.525 79.525) (width 0.2) (layer "F.Cu") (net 9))
 (segment (start 82.525 79.525) (end 82 79) (width 0.2) (layer "F.Cu") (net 9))
 (via (at 82 79) (size 0.45) (drill 0.2) (layers "F.Cu" "B.Cu") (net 9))
 (segment (start 81.5 78.5) (end 79.1 78.5) (width 0.2) (layer "B.Cu") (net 9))
 (segment (start 82 79) (end 81.5 78.5) (width 0.2) (layer "B.Cu") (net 9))
 (segment (start 80.2 84.5) (end 79.35 84.5) (width 0.2) (layer "F.Cu") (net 7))
 (segment (start 82.613292 82.934532) (end 82.547824 83) (width 0.2) (layer "F.Cu") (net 7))
 (segment (start 83.683179 79.9995) (end 83.858679 80.175) (width 0.2) (layer "F.Cu") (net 7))
 (segment (start 83.858679 80.175) (end 84.7 80.175) (width 0.2) (layer "F.Cu") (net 7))
 (segment (start 81.7 83) (end 80.2 84.5) (width 0.2) (layer "F.Cu") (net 7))
 (segment (start 82.547824 83) (end 81.7 83) (width 0.2) (layer "F.Cu") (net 7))
 (via (at 82.613292 82.934532) (size 0.45) (drill 0.2) (layers "F.Cu" "B.Cu") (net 7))
 (via (at 83.683179 79.9995) (size 0.45) (drill 0.2) (layers "F.Cu" "B.Cu") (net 7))
 (segment (start 84.029273 81.165701) (end 84.029273 80.345594) (width 0.2) (layer "B.Cu") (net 7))
 (segment (start 82.613292 82.934532) (end 82.773484 82.77434) (width 0.2) (layer "B.Cu") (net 7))
 (segment (start 82.773484 82.77434) (end 82.773484 82.42149) (width 0.2) (layer "B.Cu") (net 7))
 (segment (start 82.773484 82.42149) (end 84.029273 81.165701) (width 0.2) (layer "B.Cu") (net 7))
 (segment (start 84.029273 80.345594) (end 83.683179 79.9995) (width 0.2) (layer "B.Cu") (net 7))
 (segment (start 92.45 82.1245) (end 92.45 83.285246) (width 0.2) (layer "F.Cu") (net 13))
 (segment (start 92.45 83.285246) (end 91.010246 84.725) (width 0.2) (layer "F.Cu") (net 13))
 (segment (start 91.010246 84.725) (end 90.425 84.725) (width 0.2) (layer "F.Cu") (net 13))
 (segment (start 92.5745 82) (end 92.45 82.1245) (width 0.2) (layer "F.Cu") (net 13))
 (segment (start 94.905026 78.5) (end 95.65 78.5) (width 0.2) (layer "F.Cu") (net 13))
 (segment (start 92.082781 81.146174) (end 92.258852 81.146174) (width 0.2) (layer "F.Cu") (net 13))
 (segment (start 92.258852 81.146174) (end 94.905026 78.5) (width 0.2) (layer "F.Cu") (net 13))
 (via (at 92.5745 82) (size 0.45) (drill 0.2) (layers "F.Cu" "B.Cu") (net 13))
 (via (at 92.082781 81.146174) (size 0.45) (drill 0.2) (layers "F.Cu" "B.Cu") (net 13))
 (segment (start 92.082781 81.508281) (end 92.5745 82) (width 0.2) (layer "B.Cu") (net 13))
 (segment (start 92.082781 81.146174) (end 92.082781 81.508281) (width 0.2) (layer "B.Cu") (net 13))
 (segment (start 92.1 83.140272) (end 92.1 81.8) (width 0.2) (layer "F.Cu") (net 14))
 (segment (start 93.4 80.5) (end 95.65 80.5) (width 0.2) (layer "F.Cu") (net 14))
 (segment (start 91.165272 84.075) (end 92.1 83.140272) (width 0.2) (layer "F.Cu") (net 14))
 (segment (start 92.1 81.8) (end 93.4 80.5) (width 0.2) (layer "F.Cu") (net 14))
 (segment (start 90.425 84.075) (end 91.165272 84.075) (width 0.2) (layer "F.Cu") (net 14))
 (segment (start 79.975 84.5) (end 79.3 84.5) (width 0.5) (layer "B.Cu") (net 12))
 (segment (start 79.3 84.5) (end 95.5 84.5) (width 0.5) (layer "B.Cu") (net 12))
 (segment (start 81.964141 81.614335) (end 83.25 82.900194) (width 0.2) (layer "F.Cu") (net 10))
 (segment (start 83.25 83.210246) (end 84.114754 84.075) (width 0.2) (layer "F.Cu") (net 10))
 (segment (start 81.964141 81.19338) (end 81.964141 81.614335) (width 0.2) (layer "F.Cu") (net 10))
 (segment (start 81.990958 80.991967) (end 81.990958 81.166563) (width 0.2) (layer "F.Cu") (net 10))
 (segment (start 83.25 82.900194) (end 83.25 83.210246) (width 0.2) (layer "F.Cu") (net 10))
 (segment (start 84.114754 84.075) (end 84.7 84.075) (width 0.2) (layer "F.Cu") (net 10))
 (segment (start 81.990958 81.166563) (end 81.964141 81.19338) (width 0.2) (layer "F.Cu") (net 10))
 (via (at 81.990958 80.991967) (size 0.45) (drill 0.2) (layers "F.Cu" "B.Cu") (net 10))
 (segment (start 81.990958 80.991967) (end 81.498991 80.5) (width 0.2) (layer "B.Cu") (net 10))
 (segment (start 81.498991 80.5) (end 79.6 80.5) (width 0.2) (layer "B.Cu") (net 10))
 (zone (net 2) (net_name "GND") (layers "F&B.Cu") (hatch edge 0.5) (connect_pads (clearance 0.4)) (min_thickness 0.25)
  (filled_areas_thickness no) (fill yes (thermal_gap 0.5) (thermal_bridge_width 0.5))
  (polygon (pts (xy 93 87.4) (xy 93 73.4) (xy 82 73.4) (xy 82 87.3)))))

